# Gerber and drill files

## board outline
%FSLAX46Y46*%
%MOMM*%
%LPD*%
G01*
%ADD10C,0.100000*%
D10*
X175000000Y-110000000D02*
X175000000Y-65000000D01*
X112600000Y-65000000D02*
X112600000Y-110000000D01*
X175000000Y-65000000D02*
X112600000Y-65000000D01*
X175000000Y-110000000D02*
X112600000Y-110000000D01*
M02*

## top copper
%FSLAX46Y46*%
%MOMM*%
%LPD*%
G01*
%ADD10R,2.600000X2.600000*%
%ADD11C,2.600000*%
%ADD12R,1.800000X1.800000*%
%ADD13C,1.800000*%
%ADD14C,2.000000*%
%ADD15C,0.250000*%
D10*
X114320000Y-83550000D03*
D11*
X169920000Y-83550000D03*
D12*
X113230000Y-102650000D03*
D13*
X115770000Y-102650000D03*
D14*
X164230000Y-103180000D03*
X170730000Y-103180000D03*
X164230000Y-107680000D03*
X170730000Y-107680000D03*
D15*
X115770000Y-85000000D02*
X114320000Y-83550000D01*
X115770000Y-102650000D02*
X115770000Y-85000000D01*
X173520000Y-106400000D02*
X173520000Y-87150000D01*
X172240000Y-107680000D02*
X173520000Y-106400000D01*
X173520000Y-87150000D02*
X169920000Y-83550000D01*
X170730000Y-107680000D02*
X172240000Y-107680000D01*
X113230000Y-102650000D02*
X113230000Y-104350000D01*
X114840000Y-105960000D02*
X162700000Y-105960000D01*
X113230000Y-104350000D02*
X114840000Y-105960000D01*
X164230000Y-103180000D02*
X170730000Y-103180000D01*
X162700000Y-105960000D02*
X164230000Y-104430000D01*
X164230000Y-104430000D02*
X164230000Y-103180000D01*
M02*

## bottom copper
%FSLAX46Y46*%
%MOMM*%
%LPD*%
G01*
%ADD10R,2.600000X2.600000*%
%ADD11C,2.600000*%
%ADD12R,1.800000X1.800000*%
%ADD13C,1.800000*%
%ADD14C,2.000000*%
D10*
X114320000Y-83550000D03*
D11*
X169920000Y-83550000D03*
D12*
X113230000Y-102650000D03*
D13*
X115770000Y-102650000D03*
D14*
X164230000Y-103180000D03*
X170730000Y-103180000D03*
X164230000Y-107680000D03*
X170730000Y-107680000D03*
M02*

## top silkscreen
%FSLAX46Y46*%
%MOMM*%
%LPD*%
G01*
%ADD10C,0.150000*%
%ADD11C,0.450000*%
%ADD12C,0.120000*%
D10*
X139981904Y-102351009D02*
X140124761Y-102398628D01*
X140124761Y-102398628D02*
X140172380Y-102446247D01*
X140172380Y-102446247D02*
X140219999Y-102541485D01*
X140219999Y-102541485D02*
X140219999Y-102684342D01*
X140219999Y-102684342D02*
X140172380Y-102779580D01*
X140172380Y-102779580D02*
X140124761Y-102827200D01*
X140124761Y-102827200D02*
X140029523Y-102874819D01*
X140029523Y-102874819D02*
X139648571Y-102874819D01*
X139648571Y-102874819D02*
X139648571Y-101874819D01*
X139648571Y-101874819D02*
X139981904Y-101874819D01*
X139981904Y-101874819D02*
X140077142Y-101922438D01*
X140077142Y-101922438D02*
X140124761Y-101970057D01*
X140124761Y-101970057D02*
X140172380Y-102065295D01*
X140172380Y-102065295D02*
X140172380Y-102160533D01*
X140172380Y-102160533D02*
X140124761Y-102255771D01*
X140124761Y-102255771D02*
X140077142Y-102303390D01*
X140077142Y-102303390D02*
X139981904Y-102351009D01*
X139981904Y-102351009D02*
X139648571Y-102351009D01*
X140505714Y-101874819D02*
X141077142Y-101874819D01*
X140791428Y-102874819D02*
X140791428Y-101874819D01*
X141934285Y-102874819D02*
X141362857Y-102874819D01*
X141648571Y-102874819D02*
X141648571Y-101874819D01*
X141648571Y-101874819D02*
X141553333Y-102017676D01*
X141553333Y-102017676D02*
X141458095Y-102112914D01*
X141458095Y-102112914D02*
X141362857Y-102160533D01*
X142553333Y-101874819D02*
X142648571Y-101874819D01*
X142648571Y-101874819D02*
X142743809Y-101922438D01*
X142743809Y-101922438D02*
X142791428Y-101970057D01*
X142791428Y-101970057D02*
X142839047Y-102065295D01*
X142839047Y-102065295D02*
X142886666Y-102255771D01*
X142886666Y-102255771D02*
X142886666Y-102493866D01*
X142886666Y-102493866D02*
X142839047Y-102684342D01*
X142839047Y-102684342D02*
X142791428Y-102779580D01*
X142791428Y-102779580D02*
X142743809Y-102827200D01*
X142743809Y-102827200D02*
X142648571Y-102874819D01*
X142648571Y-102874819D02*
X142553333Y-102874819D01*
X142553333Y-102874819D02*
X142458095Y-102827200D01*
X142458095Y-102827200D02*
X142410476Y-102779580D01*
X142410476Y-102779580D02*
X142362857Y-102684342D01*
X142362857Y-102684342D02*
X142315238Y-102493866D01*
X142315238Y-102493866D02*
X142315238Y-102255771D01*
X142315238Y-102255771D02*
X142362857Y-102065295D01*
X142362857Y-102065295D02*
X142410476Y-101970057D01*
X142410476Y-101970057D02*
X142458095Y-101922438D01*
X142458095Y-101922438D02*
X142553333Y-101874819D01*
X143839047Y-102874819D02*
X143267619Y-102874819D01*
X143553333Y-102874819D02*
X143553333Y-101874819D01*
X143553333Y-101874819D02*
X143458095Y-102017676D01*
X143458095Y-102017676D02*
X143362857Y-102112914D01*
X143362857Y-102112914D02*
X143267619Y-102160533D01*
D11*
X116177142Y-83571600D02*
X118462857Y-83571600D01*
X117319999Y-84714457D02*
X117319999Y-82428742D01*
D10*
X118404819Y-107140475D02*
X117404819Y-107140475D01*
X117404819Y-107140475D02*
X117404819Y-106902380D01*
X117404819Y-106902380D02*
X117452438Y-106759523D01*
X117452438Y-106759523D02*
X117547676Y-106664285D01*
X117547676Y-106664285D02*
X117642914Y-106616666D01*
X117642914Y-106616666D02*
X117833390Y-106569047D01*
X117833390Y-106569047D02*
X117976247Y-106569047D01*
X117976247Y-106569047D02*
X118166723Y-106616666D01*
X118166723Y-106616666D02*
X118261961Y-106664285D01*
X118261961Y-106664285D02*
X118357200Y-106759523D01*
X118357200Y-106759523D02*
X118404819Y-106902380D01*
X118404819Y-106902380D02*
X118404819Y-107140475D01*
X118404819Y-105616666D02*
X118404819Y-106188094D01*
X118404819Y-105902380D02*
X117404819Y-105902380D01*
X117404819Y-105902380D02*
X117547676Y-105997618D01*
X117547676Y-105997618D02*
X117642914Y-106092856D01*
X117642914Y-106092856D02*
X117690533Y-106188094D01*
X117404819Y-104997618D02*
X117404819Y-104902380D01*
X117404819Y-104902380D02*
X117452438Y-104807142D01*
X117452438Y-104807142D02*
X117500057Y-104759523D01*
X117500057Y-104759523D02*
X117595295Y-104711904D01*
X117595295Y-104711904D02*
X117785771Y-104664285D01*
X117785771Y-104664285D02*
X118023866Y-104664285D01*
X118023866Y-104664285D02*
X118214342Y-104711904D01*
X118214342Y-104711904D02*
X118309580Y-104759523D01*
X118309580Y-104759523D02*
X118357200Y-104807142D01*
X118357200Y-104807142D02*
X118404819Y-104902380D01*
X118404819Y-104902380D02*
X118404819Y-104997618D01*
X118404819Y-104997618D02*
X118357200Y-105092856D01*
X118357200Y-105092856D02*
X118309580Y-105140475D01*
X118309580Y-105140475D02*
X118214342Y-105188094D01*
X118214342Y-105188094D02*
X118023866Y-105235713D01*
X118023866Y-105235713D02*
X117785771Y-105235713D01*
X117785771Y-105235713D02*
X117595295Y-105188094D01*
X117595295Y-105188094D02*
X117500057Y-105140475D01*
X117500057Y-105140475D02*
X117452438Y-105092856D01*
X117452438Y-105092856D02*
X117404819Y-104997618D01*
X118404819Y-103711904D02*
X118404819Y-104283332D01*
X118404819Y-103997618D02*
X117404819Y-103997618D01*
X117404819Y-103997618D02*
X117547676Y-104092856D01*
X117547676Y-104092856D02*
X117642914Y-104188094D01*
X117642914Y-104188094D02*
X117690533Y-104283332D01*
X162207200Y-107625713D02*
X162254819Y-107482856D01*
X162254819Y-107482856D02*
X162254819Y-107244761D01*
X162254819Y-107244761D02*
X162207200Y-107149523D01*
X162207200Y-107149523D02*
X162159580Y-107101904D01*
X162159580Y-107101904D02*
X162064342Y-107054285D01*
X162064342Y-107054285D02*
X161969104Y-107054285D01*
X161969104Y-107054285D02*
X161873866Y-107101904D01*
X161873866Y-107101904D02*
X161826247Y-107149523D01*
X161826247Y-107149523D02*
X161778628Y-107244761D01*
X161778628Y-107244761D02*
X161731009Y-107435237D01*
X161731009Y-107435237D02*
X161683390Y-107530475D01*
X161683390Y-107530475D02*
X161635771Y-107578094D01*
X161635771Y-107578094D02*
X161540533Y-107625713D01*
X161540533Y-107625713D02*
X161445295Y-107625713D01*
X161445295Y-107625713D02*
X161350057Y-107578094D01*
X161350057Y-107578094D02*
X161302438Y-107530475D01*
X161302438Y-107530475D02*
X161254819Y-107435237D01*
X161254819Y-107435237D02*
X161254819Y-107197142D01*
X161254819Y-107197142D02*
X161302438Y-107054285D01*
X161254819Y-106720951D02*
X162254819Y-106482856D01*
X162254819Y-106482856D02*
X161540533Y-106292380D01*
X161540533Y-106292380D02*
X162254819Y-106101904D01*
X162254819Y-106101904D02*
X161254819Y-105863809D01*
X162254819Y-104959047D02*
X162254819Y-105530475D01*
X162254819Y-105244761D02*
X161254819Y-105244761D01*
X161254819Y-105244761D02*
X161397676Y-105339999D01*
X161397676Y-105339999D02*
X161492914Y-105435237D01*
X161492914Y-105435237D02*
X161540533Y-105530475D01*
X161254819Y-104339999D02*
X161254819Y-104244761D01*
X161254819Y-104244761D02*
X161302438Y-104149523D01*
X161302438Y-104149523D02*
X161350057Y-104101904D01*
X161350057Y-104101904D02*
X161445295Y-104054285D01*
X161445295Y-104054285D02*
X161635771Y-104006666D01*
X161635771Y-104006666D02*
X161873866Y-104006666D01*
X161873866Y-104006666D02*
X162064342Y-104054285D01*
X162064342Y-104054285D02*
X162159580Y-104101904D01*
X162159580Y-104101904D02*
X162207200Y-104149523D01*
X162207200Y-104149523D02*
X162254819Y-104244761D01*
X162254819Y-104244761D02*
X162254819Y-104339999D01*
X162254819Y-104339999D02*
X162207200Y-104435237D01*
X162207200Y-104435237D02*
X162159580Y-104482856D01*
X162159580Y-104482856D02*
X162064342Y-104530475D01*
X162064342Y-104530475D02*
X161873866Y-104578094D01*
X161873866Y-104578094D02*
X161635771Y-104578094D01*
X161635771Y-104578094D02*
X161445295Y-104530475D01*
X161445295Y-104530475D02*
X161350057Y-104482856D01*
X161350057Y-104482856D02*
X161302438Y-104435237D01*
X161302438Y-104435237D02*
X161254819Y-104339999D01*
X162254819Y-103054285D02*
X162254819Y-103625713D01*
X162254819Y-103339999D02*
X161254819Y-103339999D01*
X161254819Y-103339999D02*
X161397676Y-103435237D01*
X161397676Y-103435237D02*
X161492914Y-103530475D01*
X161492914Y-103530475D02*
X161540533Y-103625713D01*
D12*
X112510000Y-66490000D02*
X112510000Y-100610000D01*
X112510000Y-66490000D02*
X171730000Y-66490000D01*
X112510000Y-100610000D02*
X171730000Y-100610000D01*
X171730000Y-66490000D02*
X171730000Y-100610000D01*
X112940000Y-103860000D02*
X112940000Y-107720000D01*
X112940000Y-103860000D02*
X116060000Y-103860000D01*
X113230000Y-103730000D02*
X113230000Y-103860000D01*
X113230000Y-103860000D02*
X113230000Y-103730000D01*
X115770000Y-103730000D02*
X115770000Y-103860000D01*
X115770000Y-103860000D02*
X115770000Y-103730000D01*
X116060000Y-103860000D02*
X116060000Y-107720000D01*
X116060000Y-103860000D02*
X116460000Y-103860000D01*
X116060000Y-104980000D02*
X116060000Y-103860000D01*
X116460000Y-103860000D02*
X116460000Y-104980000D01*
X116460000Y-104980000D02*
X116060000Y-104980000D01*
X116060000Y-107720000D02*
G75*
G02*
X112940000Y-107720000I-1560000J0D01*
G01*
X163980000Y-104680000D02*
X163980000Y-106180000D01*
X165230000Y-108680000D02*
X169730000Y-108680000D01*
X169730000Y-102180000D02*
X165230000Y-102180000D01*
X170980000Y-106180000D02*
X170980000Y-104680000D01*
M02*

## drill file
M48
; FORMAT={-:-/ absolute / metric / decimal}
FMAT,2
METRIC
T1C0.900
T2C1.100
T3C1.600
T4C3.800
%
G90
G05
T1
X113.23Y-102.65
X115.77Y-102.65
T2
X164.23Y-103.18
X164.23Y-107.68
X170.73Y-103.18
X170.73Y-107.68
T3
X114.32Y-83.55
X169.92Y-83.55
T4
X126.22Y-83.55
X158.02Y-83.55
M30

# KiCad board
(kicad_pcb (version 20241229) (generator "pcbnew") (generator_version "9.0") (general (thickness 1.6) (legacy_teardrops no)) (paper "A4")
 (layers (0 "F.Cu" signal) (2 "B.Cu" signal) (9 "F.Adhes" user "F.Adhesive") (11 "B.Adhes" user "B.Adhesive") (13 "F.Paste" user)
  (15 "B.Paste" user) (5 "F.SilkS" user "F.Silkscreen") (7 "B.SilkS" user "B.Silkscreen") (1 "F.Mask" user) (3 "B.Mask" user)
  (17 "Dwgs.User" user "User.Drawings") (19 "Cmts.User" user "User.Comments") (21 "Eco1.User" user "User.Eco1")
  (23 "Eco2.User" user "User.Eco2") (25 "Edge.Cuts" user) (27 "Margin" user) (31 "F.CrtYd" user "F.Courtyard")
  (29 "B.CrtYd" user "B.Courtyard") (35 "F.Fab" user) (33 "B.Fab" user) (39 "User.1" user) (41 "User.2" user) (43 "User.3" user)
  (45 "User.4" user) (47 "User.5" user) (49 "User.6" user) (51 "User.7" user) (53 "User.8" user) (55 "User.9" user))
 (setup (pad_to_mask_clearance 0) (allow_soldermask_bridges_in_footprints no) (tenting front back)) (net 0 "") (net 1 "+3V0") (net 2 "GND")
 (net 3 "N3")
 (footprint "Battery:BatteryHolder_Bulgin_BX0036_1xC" (layer "F.Cu") (at 114.32 83.55)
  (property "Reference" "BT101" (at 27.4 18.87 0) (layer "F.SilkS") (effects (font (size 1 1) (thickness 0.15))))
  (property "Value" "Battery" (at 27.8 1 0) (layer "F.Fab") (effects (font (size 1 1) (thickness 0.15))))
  (fp_line (start -1.81 -17.06) (end -1.81 17.06) (stroke (width 0.12) (type solid)) (layer "F.SilkS"))
  (fp_line (start -1.81 -17.06) (end 57.41 -17.06) (stroke (width 0.12) (type solid)) (layer "F.SilkS"))
  (fp_line (start -1.81 17.06) (end 57.41 17.06) (stroke (width 0.12) (type solid)) (layer "F.SilkS"))
  (fp_line (start 57.41 -17.06) (end 57.41 17.06) (stroke (width 0.12) (type solid)) (layer "F.SilkS"))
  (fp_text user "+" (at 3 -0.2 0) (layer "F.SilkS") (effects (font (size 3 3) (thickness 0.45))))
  (pad "" np_thru_hole circle (at 11.9 0) (size 3.8 3.8) (drill 3.8) (layers "*.Cu" "*.Mask"))
  (pad "" np_thru_hole circle (at 43.7 0) (size 3.8 3.8) (drill 3.8) (layers "*.Cu" "*.Mask"))
  (pad "1" thru_hole rect (at 0 0) (size 2.6 2.6) (drill 1.6) (layers "*.Cu" "*.Mask") (remove_unused_layers no) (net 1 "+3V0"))
  (pad "2" thru_hole circle (at 55.6 0) (size 2.6 2.6) (drill 1.6) (layers "*.Cu" "*.Mask") (remove_unused_layers no) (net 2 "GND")))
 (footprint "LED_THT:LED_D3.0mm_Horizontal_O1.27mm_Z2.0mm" (layer "F.Cu") (at 113.23 102.65)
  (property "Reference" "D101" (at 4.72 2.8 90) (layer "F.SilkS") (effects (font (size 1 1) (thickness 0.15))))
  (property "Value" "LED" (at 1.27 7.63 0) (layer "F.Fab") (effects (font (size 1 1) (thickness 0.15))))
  (fp_line (start -0.29 1.21) (end -0.29 5.07) (stroke (width 0.12) (type solid)) (layer "F.SilkS"))
  (fp_line (start -0.29 1.21) (end 2.83 1.21) (stroke (width 0.12) (type solid)) (layer "F.SilkS"))
  (fp_line (start 0 1.08) (end 0 1.21) (stroke (width 0.12) (type solid)) (layer "F.SilkS"))
  (fp_line (start 0 1.21) (end 0 1.08) (stroke (width 0.12) (type solid)) (layer "F.SilkS"))
  (fp_line (start 2.54 1.08) (end 2.54 1.21) (stroke (width 0.12) (type solid)) (layer "F.SilkS"))
  (fp_line (start 2.54 1.21) (end 2.54 1.08) (stroke (width 0.12) (type solid)) (layer "F.SilkS"))
  (fp_line (start 2.83 1.21) (end 2.83 5.07) (stroke (width 0.12) (type solid)) (layer "F.SilkS"))
  (fp_line (start 2.83 1.21) (end 3.23 1.21) (stroke (width 0.12) (type solid)) (layer "F.SilkS"))
  (fp_line (start 2.83 2.33) (end 2.83 1.21) (stroke (width 0.12) (type solid)) (layer "F.SilkS"))
  (fp_line (start 3.23 1.21) (end 3.23 2.33) (stroke (width 0.12) (type solid)) (layer "F.SilkS"))
  (fp_line (start 3.23 2.33) (end 2.83 2.33) (stroke (width 0.12) (type solid)) (layer "F.SilkS"))
  (fp_arc (start 2.83 5.07) (mid 1.27 6.63) (end -0.29 5.07) (stroke (width 0.12) (type solid)) (layer "F.SilkS"))
  (pad "1" thru_hole rect (at 0 0) (size 1.8 1.8) (drill 0.9) (layers "*.Cu" "*.Mask") (remove_unused_layers no) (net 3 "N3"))
  (pad "2" thru_hole circle (at 2.54 0) (size 1.8 1.8) (drill 0.9) (layers "*.Cu" "*.Mask") (remove_unused_layers no) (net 1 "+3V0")))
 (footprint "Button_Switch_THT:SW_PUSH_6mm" (layer "F.Cu") (at 164.23 103.18)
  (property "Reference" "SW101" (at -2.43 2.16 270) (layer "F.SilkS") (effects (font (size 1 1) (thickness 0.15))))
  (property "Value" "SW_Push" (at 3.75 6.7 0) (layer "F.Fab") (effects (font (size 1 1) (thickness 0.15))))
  (fp_line (start -0.25 1.5) (end -0.25 3) (stroke (width 0.12) (type solid)) (layer "F.SilkS"))
  (fp_line (start 1 5.5) (end 5.5 5.5) (stroke (width 0.12) (type solid)) (layer "F.SilkS"))
  (fp_line (start 5.5 -1) (end 1 -1) (stroke (width 0.12) (type solid)) (layer "F.SilkS"))
  (fp_line (start 6.75 3) (end 6.75 1.5) (stroke (width 0.12) (type solid)) (layer "F.SilkS"))
  (pad "1" thru_hole circle (at 0 0 90) (size 2 2) (drill 1.1) (layers "*.Cu" "*.Mask") (remove_unused_layers no) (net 3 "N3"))
  (pad "1" thru_hole circle (at 6.5 0 90) (size 2 2) (drill 1.1) (layers "*.Cu" "*.Mask") (remove_unused_layers no) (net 3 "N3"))
  (pad "2" thru_hole circle (at 0 4.5 90) (size 2 2) (drill 1.1) (layers "*.Cu" "*.Mask") (remove_unused_layers no) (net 2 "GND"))
  (pad "2" thru_hole circle (at 6.5 4.5 90) (size 2 2) (drill 1.1) (layers "*.Cu" "*.Mask") (remove_unused_layers no) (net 2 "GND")))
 (gr_line (start 175 110) (end 175 65) (stroke (width 0.1) (type default)) (layer "Edge.Cuts"))
 (gr_line (start 112.6 65) (end 112.6 110) (stroke (width 0.1) (type default)) (layer "Edge.Cuts"))
 (gr_line (start 175 65) (end 112.6 65) (stroke (width 0.1) (type default)) (layer "Edge.Cuts"))
 (gr_line (start 175 110) (end 112.6 110) (stroke (width 0.1) (type default)) (layer "Edge.Cuts"))
 (segment (start 115.77 85) (end 114.32 83.55) (width 0.25) (layer "F.Cu") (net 1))
 (segment (start 115.77 102.65) (end 115.77 85) (width 0.25) (layer "F.Cu") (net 1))
 (segment (start 173.52 106.4) (end 173.52 87.15) (width 0.25) (layer "F.Cu") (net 2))
 (segment (start 172.24 107.68) (end 173.52 106.4) (width 0.25) (layer "F.Cu") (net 2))
 (segment (start 173.52 87.15) (end 169.92 83.55) (width 0.25) (layer "F.Cu") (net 2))
 (segment (start 170.73 107.68) (end 172.24 107.68) (width 0.25) (layer "F.Cu") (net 2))
 (segment (start 113.23 102.65) (end 113.23 104.35) (width 0.25) (layer "F.Cu") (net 3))
 (segment (start 114.84 105.96) (end 162.7 105.96) (width 0.25) (layer "F.Cu") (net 3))
 (segment (start 113.23 104.35) (end 114.84 105.96) (width 0.25) (layer "F.Cu") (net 3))
 (segment (start 164.23 103.18) (end 170.73 103.18) (width 0.25) (layer "F.Cu") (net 3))
 (segment (start 162.7 105.96) (end 164.23 104.43) (width 0.25) (layer "F.Cu") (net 3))
 (segment (start 164.23 104.43) (end 164.23 103.18) (width 0.25) (layer "F.Cu") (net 3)))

